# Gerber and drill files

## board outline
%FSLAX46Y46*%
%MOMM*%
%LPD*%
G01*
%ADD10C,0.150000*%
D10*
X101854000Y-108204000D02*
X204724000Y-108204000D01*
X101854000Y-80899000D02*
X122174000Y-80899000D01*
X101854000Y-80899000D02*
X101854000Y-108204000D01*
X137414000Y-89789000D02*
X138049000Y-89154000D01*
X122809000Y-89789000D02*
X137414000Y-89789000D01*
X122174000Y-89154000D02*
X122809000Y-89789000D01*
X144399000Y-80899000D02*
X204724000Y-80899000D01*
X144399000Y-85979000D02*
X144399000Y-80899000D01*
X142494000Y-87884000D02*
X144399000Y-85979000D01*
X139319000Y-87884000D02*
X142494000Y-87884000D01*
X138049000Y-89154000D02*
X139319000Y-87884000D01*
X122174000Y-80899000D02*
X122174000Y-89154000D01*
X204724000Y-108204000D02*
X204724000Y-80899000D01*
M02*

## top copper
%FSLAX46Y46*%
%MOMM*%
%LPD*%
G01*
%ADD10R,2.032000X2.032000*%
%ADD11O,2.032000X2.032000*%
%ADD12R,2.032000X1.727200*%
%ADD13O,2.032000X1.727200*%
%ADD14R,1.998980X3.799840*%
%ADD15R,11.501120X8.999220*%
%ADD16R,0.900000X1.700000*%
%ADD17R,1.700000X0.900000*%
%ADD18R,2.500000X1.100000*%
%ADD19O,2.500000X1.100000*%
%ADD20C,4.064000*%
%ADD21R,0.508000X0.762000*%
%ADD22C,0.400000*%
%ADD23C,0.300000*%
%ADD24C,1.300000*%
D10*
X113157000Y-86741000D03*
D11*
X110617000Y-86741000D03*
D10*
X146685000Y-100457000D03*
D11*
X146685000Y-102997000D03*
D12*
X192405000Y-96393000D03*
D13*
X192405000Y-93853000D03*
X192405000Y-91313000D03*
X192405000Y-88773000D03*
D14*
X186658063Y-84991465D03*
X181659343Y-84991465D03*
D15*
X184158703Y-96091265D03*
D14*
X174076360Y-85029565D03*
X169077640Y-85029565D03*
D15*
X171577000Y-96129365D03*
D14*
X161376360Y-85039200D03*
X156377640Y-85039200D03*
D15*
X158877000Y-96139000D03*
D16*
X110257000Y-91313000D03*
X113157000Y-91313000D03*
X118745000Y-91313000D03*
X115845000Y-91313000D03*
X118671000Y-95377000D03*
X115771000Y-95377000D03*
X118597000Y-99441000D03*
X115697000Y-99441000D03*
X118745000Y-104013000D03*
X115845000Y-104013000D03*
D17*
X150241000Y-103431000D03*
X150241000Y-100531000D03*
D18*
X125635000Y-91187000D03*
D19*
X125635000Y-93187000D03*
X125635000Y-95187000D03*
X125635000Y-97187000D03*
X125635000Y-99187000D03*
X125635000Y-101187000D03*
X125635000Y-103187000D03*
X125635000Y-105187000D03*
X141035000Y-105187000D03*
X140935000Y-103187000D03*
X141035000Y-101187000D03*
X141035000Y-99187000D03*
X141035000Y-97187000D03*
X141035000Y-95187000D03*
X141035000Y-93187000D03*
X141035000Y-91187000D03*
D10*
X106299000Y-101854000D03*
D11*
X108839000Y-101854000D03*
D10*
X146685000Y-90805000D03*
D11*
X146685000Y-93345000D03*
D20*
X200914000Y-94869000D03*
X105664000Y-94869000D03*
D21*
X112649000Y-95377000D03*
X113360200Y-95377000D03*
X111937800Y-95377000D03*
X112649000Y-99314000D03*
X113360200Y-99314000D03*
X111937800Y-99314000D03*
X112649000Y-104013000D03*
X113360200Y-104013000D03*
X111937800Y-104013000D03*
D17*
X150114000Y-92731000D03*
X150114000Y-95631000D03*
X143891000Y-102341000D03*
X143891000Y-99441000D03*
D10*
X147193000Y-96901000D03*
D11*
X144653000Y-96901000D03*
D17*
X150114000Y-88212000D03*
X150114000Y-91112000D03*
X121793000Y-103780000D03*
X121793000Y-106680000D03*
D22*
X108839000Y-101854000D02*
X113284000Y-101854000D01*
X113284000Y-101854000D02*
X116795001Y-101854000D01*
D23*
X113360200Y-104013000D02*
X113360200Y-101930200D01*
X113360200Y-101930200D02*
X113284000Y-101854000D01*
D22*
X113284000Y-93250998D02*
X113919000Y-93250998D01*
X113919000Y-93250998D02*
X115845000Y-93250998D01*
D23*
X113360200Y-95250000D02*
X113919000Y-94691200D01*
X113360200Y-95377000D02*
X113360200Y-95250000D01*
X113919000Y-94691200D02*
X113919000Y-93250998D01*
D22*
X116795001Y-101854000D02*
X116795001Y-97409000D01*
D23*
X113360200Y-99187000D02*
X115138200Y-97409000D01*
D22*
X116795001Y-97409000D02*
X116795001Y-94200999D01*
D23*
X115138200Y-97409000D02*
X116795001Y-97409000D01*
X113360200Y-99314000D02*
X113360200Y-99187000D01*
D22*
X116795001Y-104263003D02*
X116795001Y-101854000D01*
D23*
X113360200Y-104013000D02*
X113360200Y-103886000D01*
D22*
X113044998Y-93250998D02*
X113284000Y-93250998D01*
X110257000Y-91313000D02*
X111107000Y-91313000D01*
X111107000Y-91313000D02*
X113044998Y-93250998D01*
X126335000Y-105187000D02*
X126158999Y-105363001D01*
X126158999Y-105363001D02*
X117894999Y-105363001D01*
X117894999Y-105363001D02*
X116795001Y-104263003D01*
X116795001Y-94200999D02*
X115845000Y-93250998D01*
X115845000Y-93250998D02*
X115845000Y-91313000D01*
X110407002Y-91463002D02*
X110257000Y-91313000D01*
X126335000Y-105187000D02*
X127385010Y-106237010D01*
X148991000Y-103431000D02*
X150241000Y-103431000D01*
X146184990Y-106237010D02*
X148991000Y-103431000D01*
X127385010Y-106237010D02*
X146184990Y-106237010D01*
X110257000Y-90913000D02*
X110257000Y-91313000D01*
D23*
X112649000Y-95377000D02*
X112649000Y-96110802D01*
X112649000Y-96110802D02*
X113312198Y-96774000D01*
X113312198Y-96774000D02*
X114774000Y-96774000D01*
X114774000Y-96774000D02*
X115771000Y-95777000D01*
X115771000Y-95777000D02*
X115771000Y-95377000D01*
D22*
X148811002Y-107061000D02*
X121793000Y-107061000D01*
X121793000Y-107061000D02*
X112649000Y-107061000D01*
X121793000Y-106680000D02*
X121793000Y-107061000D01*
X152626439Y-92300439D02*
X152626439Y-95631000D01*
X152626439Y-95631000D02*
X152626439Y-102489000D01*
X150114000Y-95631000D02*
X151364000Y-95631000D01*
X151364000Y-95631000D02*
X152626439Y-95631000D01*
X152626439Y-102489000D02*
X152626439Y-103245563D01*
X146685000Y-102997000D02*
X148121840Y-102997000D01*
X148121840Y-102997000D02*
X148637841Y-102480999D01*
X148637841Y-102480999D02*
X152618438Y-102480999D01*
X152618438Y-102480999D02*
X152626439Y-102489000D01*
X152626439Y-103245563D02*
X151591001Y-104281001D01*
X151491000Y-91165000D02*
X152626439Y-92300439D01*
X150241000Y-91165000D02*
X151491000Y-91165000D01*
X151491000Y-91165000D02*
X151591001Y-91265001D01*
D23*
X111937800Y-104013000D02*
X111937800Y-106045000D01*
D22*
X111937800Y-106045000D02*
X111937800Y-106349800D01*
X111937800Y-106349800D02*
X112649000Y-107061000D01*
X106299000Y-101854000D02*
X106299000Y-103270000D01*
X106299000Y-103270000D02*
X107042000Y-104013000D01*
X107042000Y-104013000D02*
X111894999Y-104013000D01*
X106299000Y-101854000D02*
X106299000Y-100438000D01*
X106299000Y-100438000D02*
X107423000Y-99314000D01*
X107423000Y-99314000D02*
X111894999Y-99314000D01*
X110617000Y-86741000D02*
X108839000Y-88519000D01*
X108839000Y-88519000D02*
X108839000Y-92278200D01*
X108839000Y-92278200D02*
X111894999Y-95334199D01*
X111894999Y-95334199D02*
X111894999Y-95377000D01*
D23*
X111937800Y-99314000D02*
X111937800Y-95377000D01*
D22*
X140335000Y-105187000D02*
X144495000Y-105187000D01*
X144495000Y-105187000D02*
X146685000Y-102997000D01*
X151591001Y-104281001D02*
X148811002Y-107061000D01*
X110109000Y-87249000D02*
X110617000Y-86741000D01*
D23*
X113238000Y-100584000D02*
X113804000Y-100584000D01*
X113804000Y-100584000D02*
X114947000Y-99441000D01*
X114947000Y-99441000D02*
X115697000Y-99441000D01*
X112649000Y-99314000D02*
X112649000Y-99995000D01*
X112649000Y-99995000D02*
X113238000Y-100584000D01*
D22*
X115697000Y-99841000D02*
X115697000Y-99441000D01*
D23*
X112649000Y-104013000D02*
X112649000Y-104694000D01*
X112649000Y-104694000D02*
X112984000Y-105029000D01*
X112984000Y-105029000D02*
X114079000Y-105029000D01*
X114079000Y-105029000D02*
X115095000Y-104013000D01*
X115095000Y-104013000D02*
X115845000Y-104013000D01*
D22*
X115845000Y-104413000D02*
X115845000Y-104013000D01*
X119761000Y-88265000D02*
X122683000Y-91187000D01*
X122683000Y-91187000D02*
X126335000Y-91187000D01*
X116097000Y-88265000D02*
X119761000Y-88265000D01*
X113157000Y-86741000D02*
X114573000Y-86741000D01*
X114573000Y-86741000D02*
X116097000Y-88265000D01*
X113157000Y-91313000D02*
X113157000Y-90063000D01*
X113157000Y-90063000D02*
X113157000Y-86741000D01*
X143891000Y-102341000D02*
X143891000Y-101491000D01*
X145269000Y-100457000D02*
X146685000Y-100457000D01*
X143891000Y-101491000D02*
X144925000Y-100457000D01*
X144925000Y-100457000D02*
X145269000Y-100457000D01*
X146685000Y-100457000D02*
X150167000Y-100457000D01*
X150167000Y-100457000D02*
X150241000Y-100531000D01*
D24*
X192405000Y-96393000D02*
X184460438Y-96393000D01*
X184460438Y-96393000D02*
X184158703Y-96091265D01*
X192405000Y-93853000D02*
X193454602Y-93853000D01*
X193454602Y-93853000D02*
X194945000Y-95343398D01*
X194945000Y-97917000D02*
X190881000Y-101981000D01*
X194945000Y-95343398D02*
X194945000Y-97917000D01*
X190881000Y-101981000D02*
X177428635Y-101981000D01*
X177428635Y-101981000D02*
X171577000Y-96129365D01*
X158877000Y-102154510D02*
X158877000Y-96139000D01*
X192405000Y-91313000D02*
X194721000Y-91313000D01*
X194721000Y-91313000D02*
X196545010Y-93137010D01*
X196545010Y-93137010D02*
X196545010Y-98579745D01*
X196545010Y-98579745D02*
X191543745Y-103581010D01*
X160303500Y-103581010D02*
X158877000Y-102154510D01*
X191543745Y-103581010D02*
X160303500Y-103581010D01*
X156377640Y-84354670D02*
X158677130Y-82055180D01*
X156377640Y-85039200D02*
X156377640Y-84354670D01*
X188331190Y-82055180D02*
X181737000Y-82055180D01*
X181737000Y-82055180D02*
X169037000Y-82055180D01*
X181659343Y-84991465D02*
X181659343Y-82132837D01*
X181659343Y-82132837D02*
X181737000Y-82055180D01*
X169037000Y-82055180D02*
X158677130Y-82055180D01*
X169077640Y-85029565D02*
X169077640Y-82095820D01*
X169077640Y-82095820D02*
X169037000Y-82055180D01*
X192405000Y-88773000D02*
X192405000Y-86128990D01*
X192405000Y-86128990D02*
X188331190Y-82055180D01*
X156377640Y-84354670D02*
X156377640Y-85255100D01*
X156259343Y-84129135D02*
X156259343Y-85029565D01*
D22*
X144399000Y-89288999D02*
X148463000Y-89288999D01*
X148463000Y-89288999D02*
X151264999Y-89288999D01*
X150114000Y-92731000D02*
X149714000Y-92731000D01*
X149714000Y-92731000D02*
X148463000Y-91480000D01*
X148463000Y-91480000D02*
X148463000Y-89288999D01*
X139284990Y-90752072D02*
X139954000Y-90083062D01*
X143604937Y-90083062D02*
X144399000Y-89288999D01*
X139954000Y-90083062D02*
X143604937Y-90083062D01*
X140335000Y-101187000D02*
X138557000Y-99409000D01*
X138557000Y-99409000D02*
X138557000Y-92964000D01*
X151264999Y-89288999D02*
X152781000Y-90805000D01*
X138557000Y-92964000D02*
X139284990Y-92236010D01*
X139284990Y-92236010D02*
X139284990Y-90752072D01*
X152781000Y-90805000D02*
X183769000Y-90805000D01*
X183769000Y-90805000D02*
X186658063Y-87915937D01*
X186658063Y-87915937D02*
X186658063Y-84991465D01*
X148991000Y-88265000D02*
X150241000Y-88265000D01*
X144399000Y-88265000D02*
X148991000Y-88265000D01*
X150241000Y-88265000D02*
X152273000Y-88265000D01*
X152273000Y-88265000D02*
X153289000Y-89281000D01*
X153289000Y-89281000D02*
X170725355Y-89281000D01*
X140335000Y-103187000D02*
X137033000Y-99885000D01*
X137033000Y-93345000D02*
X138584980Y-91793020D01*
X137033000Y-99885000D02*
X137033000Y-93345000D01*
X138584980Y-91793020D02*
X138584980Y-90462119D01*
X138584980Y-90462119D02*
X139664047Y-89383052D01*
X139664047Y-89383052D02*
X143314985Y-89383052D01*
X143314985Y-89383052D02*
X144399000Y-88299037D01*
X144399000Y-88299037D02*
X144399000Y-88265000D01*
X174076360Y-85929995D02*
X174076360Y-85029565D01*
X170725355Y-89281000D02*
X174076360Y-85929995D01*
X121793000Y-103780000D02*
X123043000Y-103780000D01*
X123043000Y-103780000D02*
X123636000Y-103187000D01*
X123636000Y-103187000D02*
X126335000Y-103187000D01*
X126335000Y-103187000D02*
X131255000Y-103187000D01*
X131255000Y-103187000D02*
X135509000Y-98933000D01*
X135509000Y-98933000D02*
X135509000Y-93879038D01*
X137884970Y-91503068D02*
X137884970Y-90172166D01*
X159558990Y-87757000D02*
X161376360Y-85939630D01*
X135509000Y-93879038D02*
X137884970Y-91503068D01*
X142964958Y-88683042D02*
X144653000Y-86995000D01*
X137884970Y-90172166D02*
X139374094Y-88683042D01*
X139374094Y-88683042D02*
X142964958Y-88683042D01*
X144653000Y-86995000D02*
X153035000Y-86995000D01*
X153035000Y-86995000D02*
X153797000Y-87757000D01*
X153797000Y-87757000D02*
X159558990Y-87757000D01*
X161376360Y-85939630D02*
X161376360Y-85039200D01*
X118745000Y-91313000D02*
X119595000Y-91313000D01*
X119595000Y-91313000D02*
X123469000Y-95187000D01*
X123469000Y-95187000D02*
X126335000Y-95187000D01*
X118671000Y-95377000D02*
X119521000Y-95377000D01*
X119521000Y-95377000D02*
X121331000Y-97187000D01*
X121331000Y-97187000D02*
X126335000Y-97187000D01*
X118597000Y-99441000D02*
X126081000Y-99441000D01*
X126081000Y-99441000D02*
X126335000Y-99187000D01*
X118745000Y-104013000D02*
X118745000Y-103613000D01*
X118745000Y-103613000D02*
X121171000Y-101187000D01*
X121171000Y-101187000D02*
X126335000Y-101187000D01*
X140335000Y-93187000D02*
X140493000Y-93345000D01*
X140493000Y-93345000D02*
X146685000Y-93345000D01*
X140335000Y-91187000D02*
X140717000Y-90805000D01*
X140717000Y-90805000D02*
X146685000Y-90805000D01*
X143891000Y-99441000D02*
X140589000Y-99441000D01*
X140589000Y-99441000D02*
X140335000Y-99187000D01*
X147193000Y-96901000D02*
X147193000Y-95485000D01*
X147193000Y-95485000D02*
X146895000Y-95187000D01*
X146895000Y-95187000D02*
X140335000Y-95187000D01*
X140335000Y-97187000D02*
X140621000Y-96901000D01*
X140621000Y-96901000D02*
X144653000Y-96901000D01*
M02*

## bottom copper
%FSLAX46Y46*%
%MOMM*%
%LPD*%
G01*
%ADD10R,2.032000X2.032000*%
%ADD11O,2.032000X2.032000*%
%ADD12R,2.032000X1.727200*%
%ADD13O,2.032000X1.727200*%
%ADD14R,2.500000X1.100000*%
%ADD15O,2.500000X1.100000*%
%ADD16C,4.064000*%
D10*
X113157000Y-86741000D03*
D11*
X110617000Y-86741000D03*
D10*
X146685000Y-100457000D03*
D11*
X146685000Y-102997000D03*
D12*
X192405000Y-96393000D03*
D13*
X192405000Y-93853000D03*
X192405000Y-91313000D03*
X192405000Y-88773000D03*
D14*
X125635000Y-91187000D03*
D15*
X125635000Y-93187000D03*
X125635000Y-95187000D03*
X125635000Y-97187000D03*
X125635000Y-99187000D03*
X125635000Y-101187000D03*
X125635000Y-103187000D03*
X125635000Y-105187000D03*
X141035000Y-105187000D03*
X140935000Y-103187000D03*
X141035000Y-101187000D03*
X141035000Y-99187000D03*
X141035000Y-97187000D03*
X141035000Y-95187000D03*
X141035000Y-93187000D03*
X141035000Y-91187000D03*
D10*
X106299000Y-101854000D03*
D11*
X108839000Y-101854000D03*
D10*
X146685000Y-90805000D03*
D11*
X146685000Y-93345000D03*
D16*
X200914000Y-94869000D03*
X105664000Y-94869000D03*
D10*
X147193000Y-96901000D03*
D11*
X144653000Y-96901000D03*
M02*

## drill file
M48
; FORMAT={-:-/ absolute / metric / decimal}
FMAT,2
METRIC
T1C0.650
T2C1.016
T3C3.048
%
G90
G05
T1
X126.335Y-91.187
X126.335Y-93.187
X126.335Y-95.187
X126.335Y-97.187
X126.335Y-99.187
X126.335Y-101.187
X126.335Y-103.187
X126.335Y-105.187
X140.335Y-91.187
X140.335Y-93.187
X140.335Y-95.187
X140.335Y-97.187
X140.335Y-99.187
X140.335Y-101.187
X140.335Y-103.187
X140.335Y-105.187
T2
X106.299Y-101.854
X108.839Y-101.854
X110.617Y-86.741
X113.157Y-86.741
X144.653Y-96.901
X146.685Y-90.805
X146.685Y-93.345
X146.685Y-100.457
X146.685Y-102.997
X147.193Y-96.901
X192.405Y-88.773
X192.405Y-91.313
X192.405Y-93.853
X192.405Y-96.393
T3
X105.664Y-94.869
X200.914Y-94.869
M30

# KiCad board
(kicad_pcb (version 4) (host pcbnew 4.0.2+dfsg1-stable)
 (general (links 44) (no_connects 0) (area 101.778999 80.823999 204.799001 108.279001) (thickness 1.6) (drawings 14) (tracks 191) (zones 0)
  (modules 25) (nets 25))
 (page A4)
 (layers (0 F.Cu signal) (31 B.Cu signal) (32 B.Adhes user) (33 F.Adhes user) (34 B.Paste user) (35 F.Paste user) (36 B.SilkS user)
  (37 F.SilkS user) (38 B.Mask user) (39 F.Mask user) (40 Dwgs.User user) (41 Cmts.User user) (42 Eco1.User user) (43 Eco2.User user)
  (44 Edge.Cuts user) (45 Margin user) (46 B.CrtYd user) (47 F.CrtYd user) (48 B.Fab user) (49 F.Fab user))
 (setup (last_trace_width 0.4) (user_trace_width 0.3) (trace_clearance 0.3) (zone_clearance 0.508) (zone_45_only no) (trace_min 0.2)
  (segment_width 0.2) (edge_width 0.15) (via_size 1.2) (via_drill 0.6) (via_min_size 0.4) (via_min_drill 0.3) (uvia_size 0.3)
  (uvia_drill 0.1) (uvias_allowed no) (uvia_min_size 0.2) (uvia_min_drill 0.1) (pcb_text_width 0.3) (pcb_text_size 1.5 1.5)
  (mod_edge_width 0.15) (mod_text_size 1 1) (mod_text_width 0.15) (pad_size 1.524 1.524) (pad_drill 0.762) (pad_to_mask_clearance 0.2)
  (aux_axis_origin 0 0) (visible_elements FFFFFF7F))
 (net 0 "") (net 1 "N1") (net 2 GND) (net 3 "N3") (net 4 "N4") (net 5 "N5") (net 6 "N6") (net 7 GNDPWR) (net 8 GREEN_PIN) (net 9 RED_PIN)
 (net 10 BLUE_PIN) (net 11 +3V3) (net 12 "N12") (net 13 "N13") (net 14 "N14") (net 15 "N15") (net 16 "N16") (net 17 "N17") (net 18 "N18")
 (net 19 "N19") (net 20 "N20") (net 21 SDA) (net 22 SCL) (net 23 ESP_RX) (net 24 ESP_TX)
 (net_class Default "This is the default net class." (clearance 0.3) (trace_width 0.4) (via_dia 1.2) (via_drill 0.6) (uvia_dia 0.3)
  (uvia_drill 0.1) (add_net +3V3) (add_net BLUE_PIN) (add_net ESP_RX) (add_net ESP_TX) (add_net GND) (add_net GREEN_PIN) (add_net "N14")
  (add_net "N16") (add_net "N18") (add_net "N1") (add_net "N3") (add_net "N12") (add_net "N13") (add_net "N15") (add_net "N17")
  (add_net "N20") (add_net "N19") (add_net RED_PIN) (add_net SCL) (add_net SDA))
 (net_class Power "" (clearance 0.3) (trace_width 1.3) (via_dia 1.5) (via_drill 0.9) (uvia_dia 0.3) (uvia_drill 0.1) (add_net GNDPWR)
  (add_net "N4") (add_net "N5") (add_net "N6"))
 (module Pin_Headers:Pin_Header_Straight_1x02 (layer B.Cu) (at 113.157 86.741 90)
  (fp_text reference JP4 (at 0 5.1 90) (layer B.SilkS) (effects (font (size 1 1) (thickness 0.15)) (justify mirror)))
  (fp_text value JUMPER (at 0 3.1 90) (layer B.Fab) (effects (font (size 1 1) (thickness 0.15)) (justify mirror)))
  (pad 1 thru_hole rect (at 0 0 90) (size 2.032 2.032) (drill 1.016) (layers *.Cu *.Mask B.SilkS) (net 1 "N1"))
  (pad 2 thru_hole oval (at 0 -2.54 90) (size 2.032 2.032) (drill 1.016) (layers *.Cu *.Mask B.SilkS) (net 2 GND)))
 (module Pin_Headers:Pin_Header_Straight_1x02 (layer B.Cu) (at 146.685 100.457 180)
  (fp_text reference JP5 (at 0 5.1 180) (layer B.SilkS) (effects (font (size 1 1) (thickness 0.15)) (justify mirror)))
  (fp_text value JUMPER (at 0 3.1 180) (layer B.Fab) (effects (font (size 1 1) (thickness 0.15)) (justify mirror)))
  (pad 1 thru_hole rect (at 0 0 180) (size 2.032 2.032) (drill 1.016) (layers *.Cu *.Mask B.SilkS) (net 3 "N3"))
  (pad 2 thru_hole oval (at 0 -2.54 180) (size 2.032 2.032) (drill 1.016) (layers *.Cu *.Mask B.SilkS) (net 2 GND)))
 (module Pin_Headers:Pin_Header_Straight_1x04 (layer B.Cu) (at 192.405 96.393)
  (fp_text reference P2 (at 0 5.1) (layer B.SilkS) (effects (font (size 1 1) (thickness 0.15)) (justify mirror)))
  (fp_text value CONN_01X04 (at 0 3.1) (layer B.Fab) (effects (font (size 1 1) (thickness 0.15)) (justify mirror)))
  (pad 1 thru_hole rect (at 0 0) (size 2.032 1.7272) (drill 1.016) (layers *.Cu *.Mask B.SilkS) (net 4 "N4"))
  (pad 2 thru_hole oval (at 0 -2.54) (size 2.032 1.7272) (drill 1.016) (layers *.Cu *.Mask B.SilkS) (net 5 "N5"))
  (pad 3 thru_hole oval (at 0 -5.08) (size 2.032 1.7272) (drill 1.016) (layers *.Cu *.Mask B.SilkS) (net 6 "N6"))
  (pad 4 thru_hole oval (at 0 -7.62) (size 2.032 1.7272) (drill 1.016) (layers *.Cu *.Mask B.SilkS) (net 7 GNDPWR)))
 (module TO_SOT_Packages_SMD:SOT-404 (layer F.Cu) (at 184.158703 90.541365 180)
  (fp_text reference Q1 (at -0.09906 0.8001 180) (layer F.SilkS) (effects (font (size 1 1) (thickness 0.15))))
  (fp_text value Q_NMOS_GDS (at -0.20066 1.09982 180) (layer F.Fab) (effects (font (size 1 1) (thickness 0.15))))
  (pad 1 smd rect (at -2.49936 5.5499 180) (size 1.99898 3.79984) (layers F.Cu F.Paste F.Mask) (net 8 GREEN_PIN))
  (pad 3 smd rect (at 2.49936 5.5499 180) (size 1.99898 3.79984) (layers F.Cu F.Paste F.Mask) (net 7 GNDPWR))
  (pad 2 smd rect (at 0 -5.5499 180) (size 11.50112 8.99922) (layers F.Cu F.Paste F.Mask) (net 4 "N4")))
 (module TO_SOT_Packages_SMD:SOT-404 (layer F.Cu) (at 171.577 90.579465 180)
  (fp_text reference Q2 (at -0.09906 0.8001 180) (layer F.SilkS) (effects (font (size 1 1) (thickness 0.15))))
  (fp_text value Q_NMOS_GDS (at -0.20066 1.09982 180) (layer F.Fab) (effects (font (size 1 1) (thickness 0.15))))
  (pad 1 smd rect (at -2.49936 5.5499 180) (size 1.99898 3.79984) (layers F.Cu F.Paste F.Mask) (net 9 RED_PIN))
  (pad 3 smd rect (at 2.49936 5.5499 180) (size 1.99898 3.79984) (layers F.Cu F.Paste F.Mask) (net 7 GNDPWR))
  (pad 2 smd rect (at 0 -5.5499 180) (size 11.50112 8.99922) (layers F.Cu F.Paste F.Mask) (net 5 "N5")))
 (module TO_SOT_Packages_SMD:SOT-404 (layer F.Cu) (at 158.877 90.5891 180)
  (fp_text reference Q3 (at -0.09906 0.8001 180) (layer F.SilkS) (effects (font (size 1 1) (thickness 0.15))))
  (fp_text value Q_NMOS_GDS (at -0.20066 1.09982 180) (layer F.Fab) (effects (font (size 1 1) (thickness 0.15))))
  (pad 1 smd rect (at -2.49936 5.5499 180) (size 1.99898 3.79984) (layers F.Cu F.Paste F.Mask) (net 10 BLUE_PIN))
  (pad 3 smd rect (at 2.49936 5.5499 180) (size 1.99898 3.79984) (layers F.Cu F.Paste F.Mask) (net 7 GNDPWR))
  (pad 2 smd rect (at 0 -5.5499 180) (size 11.50112 8.99922) (layers F.Cu F.Paste F.Mask) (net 6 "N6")))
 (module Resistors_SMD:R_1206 (layer F.Cu) (at 111.707 91.313)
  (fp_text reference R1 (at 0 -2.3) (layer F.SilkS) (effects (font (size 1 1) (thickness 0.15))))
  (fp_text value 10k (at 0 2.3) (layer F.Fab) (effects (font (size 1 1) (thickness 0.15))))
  (pad 1 smd rect (at -1.45 0) (size 0.9 1.7) (layers F.Cu F.Paste F.Mask) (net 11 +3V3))
  (pad 2 smd rect (at 1.45 0) (size 0.9 1.7) (layers F.Cu F.Paste F.Mask) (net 1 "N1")))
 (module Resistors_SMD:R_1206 (layer F.Cu) (at 117.295 91.313 180)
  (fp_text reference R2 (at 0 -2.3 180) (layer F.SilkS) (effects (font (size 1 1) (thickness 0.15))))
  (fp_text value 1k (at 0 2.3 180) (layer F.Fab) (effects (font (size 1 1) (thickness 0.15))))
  (pad 1 smd rect (at -1.45 0 180) (size 0.9 1.7) (layers F.Cu F.Paste F.Mask) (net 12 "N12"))
  (pad 2 smd rect (at 1.45 0 180) (size 0.9 1.7) (layers F.Cu F.Paste F.Mask) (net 11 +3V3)))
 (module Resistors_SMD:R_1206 (layer F.Cu) (at 117.221 95.377 180)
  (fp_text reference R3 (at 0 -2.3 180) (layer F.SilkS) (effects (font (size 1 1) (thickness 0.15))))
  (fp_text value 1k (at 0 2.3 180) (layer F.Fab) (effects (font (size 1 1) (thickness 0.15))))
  (pad 1 smd rect (at -1.45 0 180) (size 0.9 1.7) (layers F.Cu F.Paste F.Mask) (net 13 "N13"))
  (pad 2 smd rect (at 1.45 0 180) (size 0.9 1.7) (layers F.Cu F.Paste F.Mask) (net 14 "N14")))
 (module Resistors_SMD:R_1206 (layer F.Cu) (at 117.147 99.441 180)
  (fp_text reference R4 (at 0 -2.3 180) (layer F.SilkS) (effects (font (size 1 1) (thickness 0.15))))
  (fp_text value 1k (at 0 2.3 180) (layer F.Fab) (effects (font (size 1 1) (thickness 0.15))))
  (pad 1 smd rect (at -1.45 0 180) (size 0.9 1.7) (layers F.Cu F.Paste F.Mask) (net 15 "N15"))
  (pad 2 smd rect (at 1.45 0 180) (size 0.9 1.7) (layers F.Cu F.Paste F.Mask) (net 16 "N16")))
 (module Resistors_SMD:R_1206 (layer F.Cu) (at 117.295 104.013 180)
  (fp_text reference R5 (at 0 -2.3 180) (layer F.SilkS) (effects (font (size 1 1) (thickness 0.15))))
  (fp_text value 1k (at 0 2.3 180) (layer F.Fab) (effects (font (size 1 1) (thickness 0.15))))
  (pad 1 smd rect (at -1.45 0 180) (size 0.9 1.7) (layers F.Cu F.Paste F.Mask) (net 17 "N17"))
  (pad 2 smd rect (at 1.45 0 180) (size 0.9 1.7) (layers F.Cu F.Paste F.Mask) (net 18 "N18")))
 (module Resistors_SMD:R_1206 (layer F.Cu) (at 150.241 101.981 90)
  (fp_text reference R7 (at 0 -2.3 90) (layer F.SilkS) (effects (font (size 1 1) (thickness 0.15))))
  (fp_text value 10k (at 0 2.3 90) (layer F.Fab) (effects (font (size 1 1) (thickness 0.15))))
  (pad 1 smd rect (at -1.45 0 90) (size 0.9 1.7) (layers F.Cu F.Paste F.Mask) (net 11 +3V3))
  (pad 2 smd rect (at 1.45 0 90) (size 0.9 1.7) (layers F.Cu F.Paste F.Mask) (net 3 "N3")))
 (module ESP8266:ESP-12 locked (layer F.Cu) (at 126.335 91.187)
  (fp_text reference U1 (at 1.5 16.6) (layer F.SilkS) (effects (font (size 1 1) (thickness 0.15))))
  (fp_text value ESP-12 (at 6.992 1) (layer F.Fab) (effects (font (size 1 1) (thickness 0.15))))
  (pad 1 thru_hole rect (at 0 0) (size 2.5 1.1) (drill 0.65 (offset -0.7 0)) (layers *.Cu *.Mask F.SilkS) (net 1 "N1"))
  (pad 2 thru_hole oval (at 0 2) (size 2.5 1.1) (drill 0.65 (offset -0.7 0)) (layers *.Cu *.Mask F.SilkS) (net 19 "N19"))
  (pad 3 thru_hole oval (at 0 4) (size 2.5 1.1) (drill 0.65 (offset -0.7 0)) (layers *.Cu *.Mask F.SilkS) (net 12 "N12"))
  (pad 4 thru_hole oval (at 0 6) (size 2.5 1.1) (drill 0.65 (offset -0.7 0)) (layers *.Cu *.Mask F.SilkS) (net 13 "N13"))
  (pad 5 thru_hole oval (at 0 8) (size 2.5 1.1) (drill 0.65 (offset -0.7 0)) (layers *.Cu *.Mask F.SilkS) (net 15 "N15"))
  (pad 6 thru_hole oval (at 0 10) (size 2.5 1.1) (drill 0.65 (offset -0.7 0)) (layers *.Cu *.Mask F.SilkS) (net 17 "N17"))
  (pad 7 thru_hole oval (at 0 12) (size 2.5 1.1) (drill 0.65 (offset -0.7 0)) (layers *.Cu *.Mask F.SilkS) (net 10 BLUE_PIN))
  (pad 8 thru_hole oval (at 0 14) (size 2.5 1.1) (drill 0.65 (offset -0.7 0)) (layers *.Cu *.Mask F.SilkS) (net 11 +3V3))
  (pad 9 thru_hole oval (at 14 14) (size 2.5 1.1) (drill 0.65 (offset 0.7 0)) (layers *.Cu *.Mask F.SilkS) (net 2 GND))
  (pad 10 thru_hole oval (at 14 12) (size 2.5 1.1) (drill 0.65 (offset 0.6 0)) (layers *.Cu *.Mask F.SilkS) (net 9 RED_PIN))
  (pad 11 thru_hole oval (at 14 10) (size 2.5 1.1) (drill 0.65 (offset 0.7 0)) (layers *.Cu *.Mask F.SilkS) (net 8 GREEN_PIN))
  (pad 12 thru_hole oval (at 14 8) (size 2.5 1.1) (drill 0.65 (offset 0.7 0)) (layers *.Cu *.Mask F.SilkS) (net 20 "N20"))
  (pad 13 thru_hole oval (at 14 6) (size 2.5 1.1) (drill 0.65 (offset 0.7 0)) (layers *.Cu *.Mask F.SilkS) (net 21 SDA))
  (pad 14 thru_hole oval (at 14 4) (size 2.5 1.1) (drill 0.65 (offset 0.7 0)) (layers *.Cu *.Mask F.SilkS) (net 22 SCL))
  (pad 15 thru_hole oval (at 14 2) (size 2.5 1.1) (drill 0.65 (offset 0.7 0)) (layers *.Cu *.Mask F.SilkS) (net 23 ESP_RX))
  (pad 16 thru_hole oval (at 14 0) (size 2.5 1.1) (drill 0.65 (offset 0.7 0)) (layers *.Cu *.Mask F.SilkS) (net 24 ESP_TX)))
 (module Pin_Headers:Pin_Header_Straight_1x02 (layer B.Cu) (at 106.299 101.854 270)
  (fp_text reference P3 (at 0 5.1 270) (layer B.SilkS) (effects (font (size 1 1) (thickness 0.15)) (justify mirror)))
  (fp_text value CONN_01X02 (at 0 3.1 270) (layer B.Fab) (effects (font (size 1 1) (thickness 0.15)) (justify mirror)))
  (pad 1 thru_hole rect (at 0 0 270) (size 2.032 2.032) (drill 1.016) (layers *.Cu *.Mask B.SilkS) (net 2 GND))
  (pad 2 thru_hole oval (at 0 -2.54 270) (size 2.032 2.032) (drill 1.016) (layers *.Cu *.Mask B.SilkS) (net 11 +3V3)))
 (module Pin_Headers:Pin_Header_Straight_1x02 (layer B.Cu) (at 146.685 90.805 180)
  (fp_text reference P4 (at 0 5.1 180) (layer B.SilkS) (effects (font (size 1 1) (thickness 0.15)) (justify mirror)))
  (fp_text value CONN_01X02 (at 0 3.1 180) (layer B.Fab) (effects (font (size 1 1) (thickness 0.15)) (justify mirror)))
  (pad 1 thru_hole rect (at 0 0 180) (size 2.032 2.032) (drill 1.016) (layers *.Cu *.Mask B.SilkS) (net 24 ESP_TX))
  (pad 2 thru_hole oval (at 0 -2.54 180) (size 2.032 2.032) (drill 1.016) (layers *.Cu *.Mask B.SilkS) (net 23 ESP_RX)))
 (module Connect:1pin (layer F.Cu) (at 200.914 94.869)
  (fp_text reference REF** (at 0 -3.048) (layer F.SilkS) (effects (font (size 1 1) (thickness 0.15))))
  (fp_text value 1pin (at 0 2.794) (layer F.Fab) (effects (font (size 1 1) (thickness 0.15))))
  (pad 1 thru_hole circle (at 0 0) (size 4.064 4.064) (drill 3.048) (layers *.Cu *.Mask F.SilkS)))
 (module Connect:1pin (layer F.Cu) (at 105.664 94.869)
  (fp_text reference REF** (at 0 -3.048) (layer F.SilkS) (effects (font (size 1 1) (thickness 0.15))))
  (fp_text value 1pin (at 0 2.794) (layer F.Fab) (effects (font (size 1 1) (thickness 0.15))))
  (pad 1 thru_hole circle (at 0 0) (size 4.064 4.064) (drill 3.048) (layers *.Cu *.Mask F.SilkS)))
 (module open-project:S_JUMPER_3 (layer F.Cu) (at 112.649 95.377 180)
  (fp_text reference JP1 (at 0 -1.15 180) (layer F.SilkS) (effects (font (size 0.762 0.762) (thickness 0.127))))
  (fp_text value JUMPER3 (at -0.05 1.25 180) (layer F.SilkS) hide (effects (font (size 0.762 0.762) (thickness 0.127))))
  (pad 2 smd rect (at 0 0 180) (size 0.508 0.762) (layers F.Cu F.Paste F.Mask) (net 14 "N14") (clearance 0.2032))
  (pad 1 smd rect (at -0.7112 0 180) (size 0.508 0.762) (layers F.Cu F.Paste F.Mask) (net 11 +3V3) (clearance 0.2032))
  (pad 3 smd rect (at 0.7112 0 180) (size 0.508 0.762) (layers F.Cu F.Paste F.Mask) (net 2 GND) (clearance 0.2032)))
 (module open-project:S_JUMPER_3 (layer F.Cu) (at 112.649 99.314 180)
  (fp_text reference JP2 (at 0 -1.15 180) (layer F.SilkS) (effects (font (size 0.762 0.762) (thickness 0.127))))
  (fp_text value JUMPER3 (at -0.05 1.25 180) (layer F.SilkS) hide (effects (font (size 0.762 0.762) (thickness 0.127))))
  (pad 2 smd rect (at 0 0 180) (size 0.508 0.762) (layers F.Cu F.Paste F.Mask) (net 16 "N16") (clearance 0.2032))
  (pad 1 smd rect (at -0.7112 0 180) (size 0.508 0.762) (layers F.Cu F.Paste F.Mask) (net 11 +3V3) (clearance 0.2032))
  (pad 3 smd rect (at 0.7112 0 180) (size 0.508 0.762) (layers F.Cu F.Paste F.Mask) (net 2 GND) (clearance 0.2032)))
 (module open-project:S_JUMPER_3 (layer F.Cu) (at 112.649 104.013 180)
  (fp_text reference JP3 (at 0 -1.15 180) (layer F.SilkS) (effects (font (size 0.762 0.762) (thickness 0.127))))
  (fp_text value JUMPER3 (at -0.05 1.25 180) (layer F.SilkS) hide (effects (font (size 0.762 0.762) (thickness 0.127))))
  (pad 2 smd rect (at 0 0 180) (size 0.508 0.762) (layers F.Cu F.Paste F.Mask) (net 18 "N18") (clearance 0.2032))
  (pad 1 smd rect (at -0.7112 0 180) (size 0.508 0.762) (layers F.Cu F.Paste F.Mask) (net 11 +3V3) (clearance 0.2032))
  (pad 3 smd rect (at 0.7112 0 180) (size 0.508 0.762) (layers F.Cu F.Paste F.Mask) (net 2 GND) (clearance 0.2032)))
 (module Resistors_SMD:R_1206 (layer F.Cu) (at 150.114 94.181 270)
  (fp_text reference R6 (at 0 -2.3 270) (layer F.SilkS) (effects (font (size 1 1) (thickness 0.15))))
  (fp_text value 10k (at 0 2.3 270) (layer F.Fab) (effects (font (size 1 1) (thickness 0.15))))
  (pad 1 smd rect (at -1.45 0 270) (size 0.9 1.7) (layers F.Cu F.Paste F.Mask) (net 8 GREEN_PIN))
  (pad 2 smd rect (at 1.45 0 270) (size 0.9 1.7) (layers F.Cu F.Paste F.Mask) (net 2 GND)))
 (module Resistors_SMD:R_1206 (layer F.Cu) (at 143.891 100.891 90)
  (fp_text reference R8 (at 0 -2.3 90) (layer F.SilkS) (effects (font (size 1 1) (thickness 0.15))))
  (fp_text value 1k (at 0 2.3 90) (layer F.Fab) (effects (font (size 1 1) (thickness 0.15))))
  (pad 1 smd rect (at -1.45 0 90) (size 0.9 1.7) (layers F.Cu F.Paste F.Mask) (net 3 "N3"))
  (pad 2 smd rect (at 1.45 0 90) (size 0.9 1.7) (layers F.Cu F.Paste F.Mask) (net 20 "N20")))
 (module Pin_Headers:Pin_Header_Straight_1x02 (layer B.Cu) (at 147.193 96.901 90)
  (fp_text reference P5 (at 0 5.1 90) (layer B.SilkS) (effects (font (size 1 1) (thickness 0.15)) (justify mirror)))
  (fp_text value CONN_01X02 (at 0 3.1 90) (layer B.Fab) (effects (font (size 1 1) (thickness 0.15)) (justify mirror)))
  (pad 1 thru_hole rect (at 0 0 90) (size 2.032 2.032) (drill 1.016) (layers *.Cu *.Mask B.SilkS) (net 22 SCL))
  (pad 2 thru_hole oval (at 0 -2.54 90) (size 2.032 2.032) (drill 1.016) (layers *.Cu *.Mask B.SilkS) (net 21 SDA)))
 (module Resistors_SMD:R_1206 (layer F.Cu) (at 150.114 89.662 270)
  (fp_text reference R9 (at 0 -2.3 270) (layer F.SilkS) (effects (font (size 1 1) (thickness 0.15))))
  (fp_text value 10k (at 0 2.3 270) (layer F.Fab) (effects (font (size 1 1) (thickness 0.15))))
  (pad 1 smd rect (at -1.45 0 270) (size 0.9 1.7) (layers F.Cu F.Paste F.Mask) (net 9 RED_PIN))
  (pad 2 smd rect (at 1.45 0 270) (size 0.9 1.7) (layers F.Cu F.Paste F.Mask) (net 2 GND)))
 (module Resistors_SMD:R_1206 (layer F.Cu) (at 121.793 105.23 270)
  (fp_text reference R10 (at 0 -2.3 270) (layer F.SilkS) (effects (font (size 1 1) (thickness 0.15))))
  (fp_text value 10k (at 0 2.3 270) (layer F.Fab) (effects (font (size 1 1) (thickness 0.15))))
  (pad 1 smd rect (at -1.45 0 270) (size 0.9 1.7) (layers F.Cu F.Paste F.Mask) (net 10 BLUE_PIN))
  (pad 2 smd rect (at 1.45 0 270) (size 0.9 1.7) (layers F.Cu F.Paste F.Mask) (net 2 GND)))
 (gr_line (start 101.854 108.204) (end 204.724 108.204) (layer Edge.Cuts) (width 0.15))
 (gr_line (start 101.854 80.899) (end 122.174 80.899) (layer Edge.Cuts) (width 0.15))
 (gr_line (start 101.854 80.899) (end 101.854 108.204) (layer Edge.Cuts) (width 0.15))
 (gr_line (start 137.414 89.789) (end 138.049 89.154) (layer Edge.Cuts) (width 0.15))
 (gr_line (start 122.809 89.789) (end 137.414 89.789) (layer Edge.Cuts) (width 0.15))
 (gr_line (start 122.174 89.154) (end 122.809 89.789) (layer Edge.Cuts) (width 0.15))
 (gr_line (start 144.399 80.899) (end 204.724 80.899) (layer Edge.Cuts) (width 0.15))
 (gr_line (start 144.399 85.979) (end 144.399 80.899) (layer Edge.Cuts) (width 0.15))
 (gr_line (start 142.494 87.884) (end 144.399 85.979) (layer Edge.Cuts) (width 0.15))
 (gr_line (start 139.319 87.884) (end 142.494 87.884) (layer Edge.Cuts) (width 0.15))
 (gr_line (start 138.049 89.154) (end 139.319 87.884) (layer Edge.Cuts) (width 0.15))
 (gr_line (start 122.174 80.899) (end 122.174 89.154) (layer Edge.Cuts) (width 0.15))
 (gr_line (start 204.724 108.204) (end 204.724 80.899) (layer Edge.Cuts) (width 0.15))
 (segment (start 108.839 101.854) (end 113.284 101.854) (width 0.4) (layer F.Cu) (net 11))
 (segment (start 113.284 101.854) (end 116.795001 101.854) (width 0.4) (layer F.Cu) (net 11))
 (segment (start 113.3602 104.013) (end 113.3602 101.9302) (width 0.3) (layer F.Cu) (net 11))
 (segment (start 113.3602 101.9302) (end 113.284 101.854) (width 0.3) (layer F.Cu) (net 11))
 (segment (start 113.284 93.250998) (end 113.919 93.250998) (width 0.4) (layer F.Cu) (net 11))
 (segment (start 113.919 93.250998) (end 115.845 93.250998) (width 0.4) (layer F.Cu) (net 11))
 (segment (start 113.3602 95.25) (end 113.919 94.6912) (width 0.3) (layer F.Cu) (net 11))
 (segment (start 113.3602 95.377) (end 113.3602 95.25) (width 0.3) (layer F.Cu) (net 11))
 (segment (start 113.919 94.6912) (end 113.919 93.250998) (width 0.3) (layer F.Cu) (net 11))
 (segment (start 116.795001 101.854) (end 116.795001 97.409) (width 0.4) (layer F.Cu) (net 11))
 (segment (start 113.3602 99.187) (end 115.1382 97.409) (width 0.3) (layer F.Cu) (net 11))
 (segment (start 116.795001 97.409) (end 116.795001 94.200999) (width 0.4) (layer F.Cu) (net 11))
 (segment (start 115.1382 97.409) (end 116.795001 97.409) (width 0.3) (layer F.Cu) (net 11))
 (segment (start 113.3602 99.314) (end 113.3602 99.187) (width 0.3) (layer F.Cu) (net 11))
 (segment (start 116.795001 104.263003) (end 116.795001 101.854) (width 0.4) (layer F.Cu) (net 11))
 (segment (start 113.3602 104.013) (end 113.3602 103.886) (width 0.3) (layer F.Cu) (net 11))
 (segment (start 113.044998 93.250998) (end 113.284 93.250998) (width 0.4) (layer F.Cu) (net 11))
 (segment (start 110.257 91.313) (end 111.107 91.313) (width 0.4) (layer F.Cu) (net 11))
 (segment (start 111.107 91.313) (end 113.044998 93.250998) (width 0.4) (layer F.Cu) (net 11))
 (segment (start 126.335 105.187) (end 126.158999 105.363001) (width 0.4) (layer F.Cu) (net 11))
 (segment (start 126.158999 105.363001) (end 117.894999 105.363001) (width 0.4) (layer F.Cu) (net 11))
 (segment (start 117.894999 105.363001) (end 116.795001 104.263003) (width 0.4) (layer F.Cu) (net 11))
 (segment (start 116.795001 94.200999) (end 115.845 93.250998) (width 0.4) (layer F.Cu) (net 11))
 (segment (start 115.845 93.250998) (end 115.845 91.313) (width 0.4) (layer F.Cu) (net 11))
 (segment (start 110.407002 91.463002) (end 110.257 91.313) (width 0.4) (layer F.Cu) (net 11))
 (segment (start 126.335 105.187) (end 127.38501 106.23701) (width 0.4) (layer F.Cu) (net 11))
 (segment (start 148.991 103.431) (end 150.241 103.431) (width 0.4) (layer F.Cu) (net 11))
 (segment (start 146.18499 106.23701) (end 148.991 103.431) (width 0.4) (layer F.Cu) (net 11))
 (segment (start 127.38501 106.23701) (end 146.18499 106.23701) (width 0.4) (layer F.Cu) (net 11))
 (segment (start 110.257 90.913) (end 110.257 91.313) (width 0.4) (layer F.Cu) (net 11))
 (segment (start 112.649 95.377) (end 112.649 96.110802) (width 0.3) (layer F.Cu) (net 14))
 (segment (start 112.649 96.110802) (end 113.312198 96.774) (width 0.3) (layer F.Cu) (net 14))
 (segment (start 113.312198 96.774) (end 114.774 96.774) (width 0.3) (layer F.Cu) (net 14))
 (segment (start 114.774 96.774) (end 115.771 95.777) (width 0.3) (layer F.Cu) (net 14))
 (segment (start 115.771 95.777) (end 115.771 95.377) (width 0.3) (layer F.Cu) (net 14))
 (segment (start 148.811002 107.061) (end 121.793 107.061) (width 0.4) (layer F.Cu) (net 2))
 (segment (start 121.793 107.061) (end 112.649 107.061) (width 0.4) (layer F.Cu) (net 2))
 (segment (start 121.793 106.68) (end 121.793 107.061) (width 0.4) (layer F.Cu) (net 2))
 (segment (start 152.626439 92.300439) (end 152.626439 95.631) (width 0.4) (layer F.Cu) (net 2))
 (segment (start 152.626439 95.631) (end 152.626439 102.489) (width 0.4) (layer F.Cu) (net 2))
 (segment (start 150.114 95.631) (end 151.364 95.631) (width 0.4) (layer F.Cu) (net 2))
 (segment (start 151.364 95.631) (end 152.626439 95.631) (width 0.4) (layer F.Cu) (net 2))
 (segment (start 152.626439 102.489) (end 152.626439 103.245563) (width 0.4) (layer F.Cu) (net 2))
 (segment (start 146.685 102.997) (end 148.12184 102.997) (width 0.4) (layer F.Cu) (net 2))
 (segment (start 148.12184 102.997) (end 148.637841 102.480999) (width 0.4) (layer F.Cu) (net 2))
 (segment (start 148.637841 102.480999) (end 152.618438 102.480999) (width 0.4) (layer F.Cu) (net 2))
 (segment (start 152.618438 102.480999) (end 152.626439 102.489) (width 0.4) (layer F.Cu) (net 2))
 (segment (start 152.626439 103.245563) (end 151.591001 104.281001) (width 0.4) (layer F.Cu) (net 2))
 (segment (start 151.491 91.165) (end 152.626439 92.300439) (width 0.4) (layer F.Cu) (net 2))
 (segment (start 150.241 91.165) (end 151.491 91.165) (width 0.4) (layer F.Cu) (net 2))
 (segment (start 151.491 91.165) (end 151.591001 91.265001) (width 0.4) (layer F.Cu) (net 2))
 (segment (start 111.9378 104.013) (end 111.9378 106.045) (width 0.3) (layer F.Cu) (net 2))
 (segment (start 111.9378 106.045) (end 111.9378 106.3498) (width 0.4) (layer F.Cu) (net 2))
 (segment (start 111.9378 106.3498) (end 112.649 107.061) (width 0.4) (layer F.Cu) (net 2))
 (segment (start 106.299 101.854) (end 106.299 103.27) (width 0.4) (layer F.Cu) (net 2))
 (segment (start 106.299 103.27) (end 107.042 104.013) (width 0.4) (layer F.Cu) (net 2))
 (segment (start 107.042 104.013) (end 111.894999 104.013) (width 0.4) (layer F.Cu) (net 2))
 (segment (start 106.299 101.854) (end 106.299 100.438) (width 0.4) (layer F.Cu) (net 2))
 (segment (start 106.299 100.438) (end 107.423 99.314) (width 0.4) (layer F.Cu) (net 2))
 (segment (start 107.423 99.314) (end 111.894999 99.314) (width 0.4) (layer F.Cu) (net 2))
 (segment (start 110.617 86.741) (end 108.839 88.519) (width 0.4) (layer F.Cu) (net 2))
 (segment (start 108.839 88.519) (end 108.839 92.2782) (width 0.4) (layer F.Cu) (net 2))
 (segment (start 108.839 92.2782) (end 111.894999 95.334199) (width 0.4) (layer F.Cu) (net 2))
 (segment (start 111.894999 95.334199) (end 111.894999 95.377) (width 0.4) (layer F.Cu) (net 2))
 (segment (start 111.9378 99.314) (end 111.9378 95.377) (width 0.3) (layer F.Cu) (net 2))
 (segment (start 140.335 105.187) (end 144.495 105.187) (width 0.4) (layer F.Cu) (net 2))
 (segment (start 144.495 105.187) (end 146.685 102.997) (width 0.4) (layer F.Cu) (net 2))
 (segment (start 151.591001 104.281001) (end 148.811002 107.061) (width 0.4) (layer F.Cu) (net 2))
 (segment (start 110.109 87.249) (end 110.617 86.741) (width 0.4) (layer F.Cu) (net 2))
 (segment (start 113.238 100.584) (end 113.804 100.584) (width 0.3) (layer F.Cu) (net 16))
 (segment (start 113.804 100.584) (end 114.947 99.441) (width 0.3) (layer F.Cu) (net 16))
 (segment (start 114.947 99.441) (end 115.697 99.441) (width 0.3) (layer F.Cu) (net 16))
 (segment (start 112.649 99.314) (end 112.649 99.995) (width 0.3) (layer F.Cu) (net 16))
 (segment (start 112.649 99.995) (end 113.238 100.584) (width 0.3) (layer F.Cu) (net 16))
 (segment (start 115.697 99.841) (end 115.697 99.441) (width 0.4) (layer F.Cu) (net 16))
 (segment (start 112.649 104.013) (end 112.649 104.694) (width 0.3) (layer F.Cu) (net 18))
 (segment (start 112.649 104.694) (end 112.984 105.029) (width 0.3) (layer F.Cu) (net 18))
 (segment (start 112.984 105.029) (end 114.079 105.029) (width 0.3) (layer F.Cu) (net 18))
 (segment (start 114.079 105.029) (end 115.095 104.013) (width 0.3) (layer F.Cu) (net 18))
 (segment (start 115.095 104.013) (end 115.845 104.013) (width 0.3) (layer F.Cu) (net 18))
 (segment (start 115.845 104.413) (end 115.845 104.013) (width 0.4) (layer F.Cu) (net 18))
 (segment (start 119.761 88.265) (end 122.683 91.187) (width 0.4) (layer F.Cu) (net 1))
 (segment (start 122.683 91.187) (end 126.335 91.187) (width 0.4) (layer F.Cu) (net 1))
 (segment (start 116.097 88.265) (end 119.761 88.265) (width 0.4) (layer F.Cu) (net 1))
 (segment (start 113.157 86.741) (end 114.573 86.741) (width 0.4) (layer F.Cu) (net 1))
 (segment (start 114.573 86.741) (end 116.097 88.265) (width 0.4) (layer F.Cu) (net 1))
 (segment (start 113.157 91.313) (end 113.157 90.063) (width 0.4) (layer F.Cu) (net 1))
 (segment (start 113.157 90.063) (end 113.157 86.741) (width 0.4) (layer F.Cu) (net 1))
 (segment (start 143.891 102.341) (end 143.891 101.491) (width 0.4) (layer F.Cu) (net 3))
 (segment (start 145.269 100.457) (end 146.685 100.457) (width 0.4) (layer F.Cu) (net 3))
 (segment (start 143.891 101.491) (end 144.925 100.457) (width 0.4) (layer F.Cu) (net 3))
 (segment (start 144.925 100.457) (end 145.269 100.457) (width 0.4) (layer F.Cu) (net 3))
 (segment (start 146.685 100.457) (end 150.167 100.457) (width 0.4) (layer F.Cu) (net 3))
 (segment (start 150.167 100.457) (end 150.241 100.531) (width 0.4) (layer F.Cu) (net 3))
 (segment (start 192.405 96.393) (end 184.460438 96.393) (width 1.3) (layer F.Cu) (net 4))
 (segment (start 184.460438 96.393) (end 184.158703 96.091265) (width 1.3) (layer F.Cu) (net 4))
 (segment (start 192.405 93.853) (end 193.454602 93.853) (width 1.3) (layer F.Cu) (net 5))
 (segment (start 193.454602 93.853) (end 194.945 95.343398) (width 1.3) (layer F.Cu) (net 5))
 (segment (start 194.945 97.917) (end 190.881 101.981) (width 1.3) (layer F.Cu) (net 5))
 (segment (start 194.945 95.343398) (end 194.945 97.917) (width 1.3) (layer F.Cu) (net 5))
 (segment (start 190.881 101.981) (end 177.428635 101.981) (width 1.3) (layer F.Cu) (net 5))
 (segment (start 177.428635 101.981) (end 171.577 96.129365) (width 1.3) (layer F.Cu) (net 5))
 (segment (start 158.877 102.15451) (end 158.877 96.139) (width 1.3) (layer F.Cu) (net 6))
 (segment (start 192.405 91.313) (end 194.721 91.313) (width 1.3) (layer F.Cu) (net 6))
 (segment (start 194.721 91.313) (end 196.54501 93.13701) (width 1.3) (layer F.Cu) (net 6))
 (segment (start 196.54501 93.13701) (end 196.54501 98.579745) (width 1.3) (layer F.Cu) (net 6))
 (segment (start 196.54501 98.579745) (end 191.543745 103.58101) (width 1.3) (layer F.Cu) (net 6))
 (segment (start 160.3035 103.58101) (end 158.877 102.15451) (width 1.3) (layer F.Cu) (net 6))
 (segment (start 191.543745 103.58101) (end 160.3035 103.58101) (width 1.3) (layer F.Cu) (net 6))
 (segment (start 156.37764 84.35467) (end 158.67713 82.05518) (width 1.3) (layer F.Cu) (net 7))
 (segment (start 156.37764 85.0392) (end 156.37764 84.35467) (width 1.3) (layer F.Cu) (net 7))
 (segment (start 188.33119 82.05518) (end 181.737 82.05518) (width 1.3) (layer F.Cu) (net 7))
 (segment (start 181.737 82.05518) (end 169.037 82.05518) (width 1.3) (layer F.Cu) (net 7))
 (segment (start 181.659343 84.991465) (end 181.659343 82.132837) (width 1.3) (layer F.Cu) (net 7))
 (segment (start 181.659343 82.132837) (end 181.737 82.05518) (width 1.3) (layer F.Cu) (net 7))
 (segment (start 169.037 82.05518) (end 158.67713 82.05518) (width 1.3) (layer F.Cu) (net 7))
 (segment (start 169.07764 85.029565) (end 169.07764 82.09582) (width 1.3) (layer F.Cu) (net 7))
 (segment (start 169.07764 82.09582) (end 169.037 82.05518) (width 1.3) (layer F.Cu) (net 7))
 (segment (start 192.405 88.773) (end 192.405 86.12899) (width 1.3) (layer F.Cu) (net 7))
 (segment (start 192.405 86.12899) (end 188.33119 82.05518) (width 1.3) (layer F.Cu) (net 7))
 (segment (start 156.37764 84.35467) (end 156.37764 85.2551) (width 1.3) (layer F.Cu) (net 7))
 (segment (start 156.259343 84.129135) (end 156.259343 85.029565) (width 1.3) (layer F.Cu) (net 7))
 (segment (start 144.399 89.288999) (end 148.463 89.288999) (width 0.4) (layer F.Cu) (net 8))
 (segment (start 148.463 89.288999) (end 151.264999 89.288999) (width 0.4) (layer F.Cu) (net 8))
 (segment (start 150.114 92.731) (end 149.714 92.731) (width 0.4) (layer F.Cu) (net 8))
 (segment (start 149.714 92.731) (end 148.463 91.48) (width 0.4) (layer F.Cu) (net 8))
 (segment (start 148.463 91.48) (end 148.463 89.288999) (width 0.4) (layer F.Cu) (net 8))
 (segment (start 139.28499 90.752072) (end 139.954 90.083062) (width 0.4) (layer F.Cu) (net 8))
 (segment (start 143.604937 90.083062) (end 144.399 89.288999) (width 0.4) (layer F.Cu) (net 8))
 (segment (start 139.954 90.083062) (end 143.604937 90.083062) (width 0.4) (layer F.Cu) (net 8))
 (segment (start 140.335 101.187) (end 138.557 99.409) (width 0.4) (layer F.Cu) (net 8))
 (segment (start 138.557 99.409) (end 138.557 92.964) (width 0.4) (layer F.Cu) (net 8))
 (segment (start 151.264999 89.288999) (end 152.781 90.805) (width 0.4) (layer F.Cu) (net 8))
 (segment (start 138.557 92.964) (end 139.28499 92.23601) (width 0.4) (layer F.Cu) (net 8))
 (segment (start 139.28499 92.23601) (end 139.28499 90.752072) (width 0.4) (layer F.Cu) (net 8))
 (segment (start 152.781 90.805) (end 183.769 90.805) (width 0.4) (layer F.Cu) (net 8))
 (segment (start 183.769 90.805) (end 186.658063 87.915937) (width 0.4) (layer F.Cu) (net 8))
 (segment (start 186.658063 87.915937) (end 186.658063 84.991465) (width 0.4) (layer F.Cu) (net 8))
 (segment (start 148.991 88.265) (end 150.241 88.265) (width 0.4) (layer F.Cu) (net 9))
 (segment (start 144.399 88.265) (end 148.991 88.265) (width 0.4) (layer F.Cu) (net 9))
 (segment (start 150.241 88.265) (end 152.273 88.265) (width 0.4) (layer F.Cu) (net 9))
 (segment (start 152.273 88.265) (end 153.289 89.281) (width 0.4) (layer F.Cu) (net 9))
 (segment (start 153.289 89.281) (end 170.725355 89.281) (width 0.4) (layer F.Cu) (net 9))
 (segment (start 140.335 103.187) (end 137.033 99.885) (width 0.4) (layer F.Cu) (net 9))
 (segment (start 137.033 93.345) (end 138.58498 91.79302) (width 0.4) (layer F.Cu) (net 9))
 (segment (start 137.033 99.885) (end 137.033 93.345) (width 0.4) (layer F.Cu) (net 9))
 (segment (start 138.58498 91.79302) (end 138.58498 90.462119) (width 0.4) (layer F.Cu) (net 9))
 (segment (start 138.58498 90.462119) (end 139.664047 89.383052) (width 0.4) (layer F.Cu) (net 9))
 (segment (start 139.664047 89.383052) (end 143.314985 89.383052) (width 0.4) (layer F.Cu) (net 9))
 (segment (start 143.314985 89.383052) (end 144.399 88.299037) (width 0.4) (layer F.Cu) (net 9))
 (segment (start 144.399 88.299037) (end 144.399 88.265) (width 0.4) (layer F.Cu) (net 9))
 (segment (start 174.07636 85.929995) (end 174.07636 85.029565) (width 0.4) (layer F.Cu) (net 9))
 (segment (start 170.725355 89.281) (end 174.07636 85.929995) (width 0.4) (layer F.Cu) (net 9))
 (segment (start 121.793 103.78) (end 123.043 103.78) (width 0.4) (layer F.Cu) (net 10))
 (segment (start 123.043 103.78) (end 123.636 103.187) (width 0.4) (layer F.Cu) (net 10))
 (segment (start 123.636 103.187) (end 126.335 103.187) (width 0.4) (layer F.Cu) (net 10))
 (segment (start 126.335 103.187) (end 131.255 103.187) (width 0.4) (layer F.Cu) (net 10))
 (segment (start 131.255 103.187) (end 135.509 98.933) (width 0.4) (layer F.Cu) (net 10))
 (segment (start 135.509 98.933) (end 135.509 93.879038) (width 0.4) (layer F.Cu) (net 10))
 (segment (start 137.88497 91.503068) (end 137.88497 90.172166) (width 0.4) (layer F.Cu) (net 10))
 (segment (start 159.55899 87.757) (end 161.37636 85.93963) (width 0.4) (layer F.Cu) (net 10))
 (segment (start 135.509 93.879038) (end 137.88497 91.503068) (width 0.4) (layer F.Cu) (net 10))
 (segment (start 142.964958 88.683042) (end 144.653 86.995) (width 0.4) (layer F.Cu) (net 10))
 (segment (start 137.88497 90.172166) (end 139.374094 88.683042) (width 0.4) (layer F.Cu) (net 10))
 (segment (start 139.374094 88.683042) (end 142.964958 88.683042) (width 0.4) (layer F.Cu) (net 10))
 (segment (start 144.653 86.995) (end 153.035 86.995) (width 0.4) (layer F.Cu) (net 10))
 (segment (start 153.035 86.995) (end 153.797 87.757) (width 0.4) (layer F.Cu) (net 10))
 (segment (start 153.797 87.757) (end 159.55899 87.757) (width 0.4) (layer F.Cu) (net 10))
 (segment (start 161.37636 85.93963) (end 161.37636 85.0392) (width 0.4) (layer F.Cu) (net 10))
 (segment (start 118.745 91.313) (end 119.595 91.313) (width 0.4) (layer F.Cu) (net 12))
 (segment (start 119.595 91.313) (end 123.469 95.187) (width 0.4) (layer F.Cu) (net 12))
 (segment (start 123.469 95.187) (end 126.335 95.187) (width 0.4) (layer F.Cu) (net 12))
 (segment (start 118.671 95.377) (end 119.521 95.377) (width 0.4) (layer F.Cu) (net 13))
 (segment (start 119.521 95.377) (end 121.331 97.187) (width 0.4) (layer F.Cu) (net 13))
 (segment (start 121.331 97.187) (end 126.335 97.187) (width 0.4) (layer F.Cu) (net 13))
 (segment (start 118.597 99.441) (end 126.081 99.441) (width 0.4) (layer F.Cu) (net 15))
 (segment (start 126.081 99.441) (end 126.335 99.187) (width 0.4) (layer F.Cu) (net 15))
 (segment (start 118.745 104.013) (end 118.745 103.613) (width 0.4) (layer F.Cu) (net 17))
 (segment (start 118.745 103.613) (end 121.171 101.187) (width 0.4) (layer F.Cu) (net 17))
 (segment (start 121.171 101.187) (end 126.335 101.187) (width 0.4) (layer F.Cu) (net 17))
 (segment (start 140.335 93.187) (end 140.493 93.345) (width 0.4) (layer F.Cu) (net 23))
 (segment (start 140.493 93.345) (end 146.685 93.345) (width 0.4) (layer F.Cu) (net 23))
 (segment (start 140.335 91.187) (end 140.717 90.805) (width 0.4) (layer F.Cu) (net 24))
 (segment (start 140.717 90.805) (end 146.685 90.805) (width 0.4) (layer F.Cu) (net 24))
 (segment (start 143.891 99.441) (end 140.589 99.441) (width 0.4) (layer F.Cu) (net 20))
 (segment (start 140.589 99.441) (end 140.335 99.187) (width 0.4) (layer F.Cu) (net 20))
 (segment (start 147.193 96.901) (end 147.193 95.485) (width 0.4) (layer F.Cu) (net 22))
 (segment (start 147.193 95.485) (end 146.895 95.187) (width 0.4) (layer F.Cu) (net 22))
 (segment (start 146.895 95.187) (end 140.335 95.187) (width 0.4) (layer F.Cu) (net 22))
 (segment (start 140.335 97.187) (end 140.621 96.901) (width 0.4) (layer F.Cu) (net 21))
 (segment (start 140.621 96.901) (end 144.653 96.901) (width 0.4) (layer F.Cu) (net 21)))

